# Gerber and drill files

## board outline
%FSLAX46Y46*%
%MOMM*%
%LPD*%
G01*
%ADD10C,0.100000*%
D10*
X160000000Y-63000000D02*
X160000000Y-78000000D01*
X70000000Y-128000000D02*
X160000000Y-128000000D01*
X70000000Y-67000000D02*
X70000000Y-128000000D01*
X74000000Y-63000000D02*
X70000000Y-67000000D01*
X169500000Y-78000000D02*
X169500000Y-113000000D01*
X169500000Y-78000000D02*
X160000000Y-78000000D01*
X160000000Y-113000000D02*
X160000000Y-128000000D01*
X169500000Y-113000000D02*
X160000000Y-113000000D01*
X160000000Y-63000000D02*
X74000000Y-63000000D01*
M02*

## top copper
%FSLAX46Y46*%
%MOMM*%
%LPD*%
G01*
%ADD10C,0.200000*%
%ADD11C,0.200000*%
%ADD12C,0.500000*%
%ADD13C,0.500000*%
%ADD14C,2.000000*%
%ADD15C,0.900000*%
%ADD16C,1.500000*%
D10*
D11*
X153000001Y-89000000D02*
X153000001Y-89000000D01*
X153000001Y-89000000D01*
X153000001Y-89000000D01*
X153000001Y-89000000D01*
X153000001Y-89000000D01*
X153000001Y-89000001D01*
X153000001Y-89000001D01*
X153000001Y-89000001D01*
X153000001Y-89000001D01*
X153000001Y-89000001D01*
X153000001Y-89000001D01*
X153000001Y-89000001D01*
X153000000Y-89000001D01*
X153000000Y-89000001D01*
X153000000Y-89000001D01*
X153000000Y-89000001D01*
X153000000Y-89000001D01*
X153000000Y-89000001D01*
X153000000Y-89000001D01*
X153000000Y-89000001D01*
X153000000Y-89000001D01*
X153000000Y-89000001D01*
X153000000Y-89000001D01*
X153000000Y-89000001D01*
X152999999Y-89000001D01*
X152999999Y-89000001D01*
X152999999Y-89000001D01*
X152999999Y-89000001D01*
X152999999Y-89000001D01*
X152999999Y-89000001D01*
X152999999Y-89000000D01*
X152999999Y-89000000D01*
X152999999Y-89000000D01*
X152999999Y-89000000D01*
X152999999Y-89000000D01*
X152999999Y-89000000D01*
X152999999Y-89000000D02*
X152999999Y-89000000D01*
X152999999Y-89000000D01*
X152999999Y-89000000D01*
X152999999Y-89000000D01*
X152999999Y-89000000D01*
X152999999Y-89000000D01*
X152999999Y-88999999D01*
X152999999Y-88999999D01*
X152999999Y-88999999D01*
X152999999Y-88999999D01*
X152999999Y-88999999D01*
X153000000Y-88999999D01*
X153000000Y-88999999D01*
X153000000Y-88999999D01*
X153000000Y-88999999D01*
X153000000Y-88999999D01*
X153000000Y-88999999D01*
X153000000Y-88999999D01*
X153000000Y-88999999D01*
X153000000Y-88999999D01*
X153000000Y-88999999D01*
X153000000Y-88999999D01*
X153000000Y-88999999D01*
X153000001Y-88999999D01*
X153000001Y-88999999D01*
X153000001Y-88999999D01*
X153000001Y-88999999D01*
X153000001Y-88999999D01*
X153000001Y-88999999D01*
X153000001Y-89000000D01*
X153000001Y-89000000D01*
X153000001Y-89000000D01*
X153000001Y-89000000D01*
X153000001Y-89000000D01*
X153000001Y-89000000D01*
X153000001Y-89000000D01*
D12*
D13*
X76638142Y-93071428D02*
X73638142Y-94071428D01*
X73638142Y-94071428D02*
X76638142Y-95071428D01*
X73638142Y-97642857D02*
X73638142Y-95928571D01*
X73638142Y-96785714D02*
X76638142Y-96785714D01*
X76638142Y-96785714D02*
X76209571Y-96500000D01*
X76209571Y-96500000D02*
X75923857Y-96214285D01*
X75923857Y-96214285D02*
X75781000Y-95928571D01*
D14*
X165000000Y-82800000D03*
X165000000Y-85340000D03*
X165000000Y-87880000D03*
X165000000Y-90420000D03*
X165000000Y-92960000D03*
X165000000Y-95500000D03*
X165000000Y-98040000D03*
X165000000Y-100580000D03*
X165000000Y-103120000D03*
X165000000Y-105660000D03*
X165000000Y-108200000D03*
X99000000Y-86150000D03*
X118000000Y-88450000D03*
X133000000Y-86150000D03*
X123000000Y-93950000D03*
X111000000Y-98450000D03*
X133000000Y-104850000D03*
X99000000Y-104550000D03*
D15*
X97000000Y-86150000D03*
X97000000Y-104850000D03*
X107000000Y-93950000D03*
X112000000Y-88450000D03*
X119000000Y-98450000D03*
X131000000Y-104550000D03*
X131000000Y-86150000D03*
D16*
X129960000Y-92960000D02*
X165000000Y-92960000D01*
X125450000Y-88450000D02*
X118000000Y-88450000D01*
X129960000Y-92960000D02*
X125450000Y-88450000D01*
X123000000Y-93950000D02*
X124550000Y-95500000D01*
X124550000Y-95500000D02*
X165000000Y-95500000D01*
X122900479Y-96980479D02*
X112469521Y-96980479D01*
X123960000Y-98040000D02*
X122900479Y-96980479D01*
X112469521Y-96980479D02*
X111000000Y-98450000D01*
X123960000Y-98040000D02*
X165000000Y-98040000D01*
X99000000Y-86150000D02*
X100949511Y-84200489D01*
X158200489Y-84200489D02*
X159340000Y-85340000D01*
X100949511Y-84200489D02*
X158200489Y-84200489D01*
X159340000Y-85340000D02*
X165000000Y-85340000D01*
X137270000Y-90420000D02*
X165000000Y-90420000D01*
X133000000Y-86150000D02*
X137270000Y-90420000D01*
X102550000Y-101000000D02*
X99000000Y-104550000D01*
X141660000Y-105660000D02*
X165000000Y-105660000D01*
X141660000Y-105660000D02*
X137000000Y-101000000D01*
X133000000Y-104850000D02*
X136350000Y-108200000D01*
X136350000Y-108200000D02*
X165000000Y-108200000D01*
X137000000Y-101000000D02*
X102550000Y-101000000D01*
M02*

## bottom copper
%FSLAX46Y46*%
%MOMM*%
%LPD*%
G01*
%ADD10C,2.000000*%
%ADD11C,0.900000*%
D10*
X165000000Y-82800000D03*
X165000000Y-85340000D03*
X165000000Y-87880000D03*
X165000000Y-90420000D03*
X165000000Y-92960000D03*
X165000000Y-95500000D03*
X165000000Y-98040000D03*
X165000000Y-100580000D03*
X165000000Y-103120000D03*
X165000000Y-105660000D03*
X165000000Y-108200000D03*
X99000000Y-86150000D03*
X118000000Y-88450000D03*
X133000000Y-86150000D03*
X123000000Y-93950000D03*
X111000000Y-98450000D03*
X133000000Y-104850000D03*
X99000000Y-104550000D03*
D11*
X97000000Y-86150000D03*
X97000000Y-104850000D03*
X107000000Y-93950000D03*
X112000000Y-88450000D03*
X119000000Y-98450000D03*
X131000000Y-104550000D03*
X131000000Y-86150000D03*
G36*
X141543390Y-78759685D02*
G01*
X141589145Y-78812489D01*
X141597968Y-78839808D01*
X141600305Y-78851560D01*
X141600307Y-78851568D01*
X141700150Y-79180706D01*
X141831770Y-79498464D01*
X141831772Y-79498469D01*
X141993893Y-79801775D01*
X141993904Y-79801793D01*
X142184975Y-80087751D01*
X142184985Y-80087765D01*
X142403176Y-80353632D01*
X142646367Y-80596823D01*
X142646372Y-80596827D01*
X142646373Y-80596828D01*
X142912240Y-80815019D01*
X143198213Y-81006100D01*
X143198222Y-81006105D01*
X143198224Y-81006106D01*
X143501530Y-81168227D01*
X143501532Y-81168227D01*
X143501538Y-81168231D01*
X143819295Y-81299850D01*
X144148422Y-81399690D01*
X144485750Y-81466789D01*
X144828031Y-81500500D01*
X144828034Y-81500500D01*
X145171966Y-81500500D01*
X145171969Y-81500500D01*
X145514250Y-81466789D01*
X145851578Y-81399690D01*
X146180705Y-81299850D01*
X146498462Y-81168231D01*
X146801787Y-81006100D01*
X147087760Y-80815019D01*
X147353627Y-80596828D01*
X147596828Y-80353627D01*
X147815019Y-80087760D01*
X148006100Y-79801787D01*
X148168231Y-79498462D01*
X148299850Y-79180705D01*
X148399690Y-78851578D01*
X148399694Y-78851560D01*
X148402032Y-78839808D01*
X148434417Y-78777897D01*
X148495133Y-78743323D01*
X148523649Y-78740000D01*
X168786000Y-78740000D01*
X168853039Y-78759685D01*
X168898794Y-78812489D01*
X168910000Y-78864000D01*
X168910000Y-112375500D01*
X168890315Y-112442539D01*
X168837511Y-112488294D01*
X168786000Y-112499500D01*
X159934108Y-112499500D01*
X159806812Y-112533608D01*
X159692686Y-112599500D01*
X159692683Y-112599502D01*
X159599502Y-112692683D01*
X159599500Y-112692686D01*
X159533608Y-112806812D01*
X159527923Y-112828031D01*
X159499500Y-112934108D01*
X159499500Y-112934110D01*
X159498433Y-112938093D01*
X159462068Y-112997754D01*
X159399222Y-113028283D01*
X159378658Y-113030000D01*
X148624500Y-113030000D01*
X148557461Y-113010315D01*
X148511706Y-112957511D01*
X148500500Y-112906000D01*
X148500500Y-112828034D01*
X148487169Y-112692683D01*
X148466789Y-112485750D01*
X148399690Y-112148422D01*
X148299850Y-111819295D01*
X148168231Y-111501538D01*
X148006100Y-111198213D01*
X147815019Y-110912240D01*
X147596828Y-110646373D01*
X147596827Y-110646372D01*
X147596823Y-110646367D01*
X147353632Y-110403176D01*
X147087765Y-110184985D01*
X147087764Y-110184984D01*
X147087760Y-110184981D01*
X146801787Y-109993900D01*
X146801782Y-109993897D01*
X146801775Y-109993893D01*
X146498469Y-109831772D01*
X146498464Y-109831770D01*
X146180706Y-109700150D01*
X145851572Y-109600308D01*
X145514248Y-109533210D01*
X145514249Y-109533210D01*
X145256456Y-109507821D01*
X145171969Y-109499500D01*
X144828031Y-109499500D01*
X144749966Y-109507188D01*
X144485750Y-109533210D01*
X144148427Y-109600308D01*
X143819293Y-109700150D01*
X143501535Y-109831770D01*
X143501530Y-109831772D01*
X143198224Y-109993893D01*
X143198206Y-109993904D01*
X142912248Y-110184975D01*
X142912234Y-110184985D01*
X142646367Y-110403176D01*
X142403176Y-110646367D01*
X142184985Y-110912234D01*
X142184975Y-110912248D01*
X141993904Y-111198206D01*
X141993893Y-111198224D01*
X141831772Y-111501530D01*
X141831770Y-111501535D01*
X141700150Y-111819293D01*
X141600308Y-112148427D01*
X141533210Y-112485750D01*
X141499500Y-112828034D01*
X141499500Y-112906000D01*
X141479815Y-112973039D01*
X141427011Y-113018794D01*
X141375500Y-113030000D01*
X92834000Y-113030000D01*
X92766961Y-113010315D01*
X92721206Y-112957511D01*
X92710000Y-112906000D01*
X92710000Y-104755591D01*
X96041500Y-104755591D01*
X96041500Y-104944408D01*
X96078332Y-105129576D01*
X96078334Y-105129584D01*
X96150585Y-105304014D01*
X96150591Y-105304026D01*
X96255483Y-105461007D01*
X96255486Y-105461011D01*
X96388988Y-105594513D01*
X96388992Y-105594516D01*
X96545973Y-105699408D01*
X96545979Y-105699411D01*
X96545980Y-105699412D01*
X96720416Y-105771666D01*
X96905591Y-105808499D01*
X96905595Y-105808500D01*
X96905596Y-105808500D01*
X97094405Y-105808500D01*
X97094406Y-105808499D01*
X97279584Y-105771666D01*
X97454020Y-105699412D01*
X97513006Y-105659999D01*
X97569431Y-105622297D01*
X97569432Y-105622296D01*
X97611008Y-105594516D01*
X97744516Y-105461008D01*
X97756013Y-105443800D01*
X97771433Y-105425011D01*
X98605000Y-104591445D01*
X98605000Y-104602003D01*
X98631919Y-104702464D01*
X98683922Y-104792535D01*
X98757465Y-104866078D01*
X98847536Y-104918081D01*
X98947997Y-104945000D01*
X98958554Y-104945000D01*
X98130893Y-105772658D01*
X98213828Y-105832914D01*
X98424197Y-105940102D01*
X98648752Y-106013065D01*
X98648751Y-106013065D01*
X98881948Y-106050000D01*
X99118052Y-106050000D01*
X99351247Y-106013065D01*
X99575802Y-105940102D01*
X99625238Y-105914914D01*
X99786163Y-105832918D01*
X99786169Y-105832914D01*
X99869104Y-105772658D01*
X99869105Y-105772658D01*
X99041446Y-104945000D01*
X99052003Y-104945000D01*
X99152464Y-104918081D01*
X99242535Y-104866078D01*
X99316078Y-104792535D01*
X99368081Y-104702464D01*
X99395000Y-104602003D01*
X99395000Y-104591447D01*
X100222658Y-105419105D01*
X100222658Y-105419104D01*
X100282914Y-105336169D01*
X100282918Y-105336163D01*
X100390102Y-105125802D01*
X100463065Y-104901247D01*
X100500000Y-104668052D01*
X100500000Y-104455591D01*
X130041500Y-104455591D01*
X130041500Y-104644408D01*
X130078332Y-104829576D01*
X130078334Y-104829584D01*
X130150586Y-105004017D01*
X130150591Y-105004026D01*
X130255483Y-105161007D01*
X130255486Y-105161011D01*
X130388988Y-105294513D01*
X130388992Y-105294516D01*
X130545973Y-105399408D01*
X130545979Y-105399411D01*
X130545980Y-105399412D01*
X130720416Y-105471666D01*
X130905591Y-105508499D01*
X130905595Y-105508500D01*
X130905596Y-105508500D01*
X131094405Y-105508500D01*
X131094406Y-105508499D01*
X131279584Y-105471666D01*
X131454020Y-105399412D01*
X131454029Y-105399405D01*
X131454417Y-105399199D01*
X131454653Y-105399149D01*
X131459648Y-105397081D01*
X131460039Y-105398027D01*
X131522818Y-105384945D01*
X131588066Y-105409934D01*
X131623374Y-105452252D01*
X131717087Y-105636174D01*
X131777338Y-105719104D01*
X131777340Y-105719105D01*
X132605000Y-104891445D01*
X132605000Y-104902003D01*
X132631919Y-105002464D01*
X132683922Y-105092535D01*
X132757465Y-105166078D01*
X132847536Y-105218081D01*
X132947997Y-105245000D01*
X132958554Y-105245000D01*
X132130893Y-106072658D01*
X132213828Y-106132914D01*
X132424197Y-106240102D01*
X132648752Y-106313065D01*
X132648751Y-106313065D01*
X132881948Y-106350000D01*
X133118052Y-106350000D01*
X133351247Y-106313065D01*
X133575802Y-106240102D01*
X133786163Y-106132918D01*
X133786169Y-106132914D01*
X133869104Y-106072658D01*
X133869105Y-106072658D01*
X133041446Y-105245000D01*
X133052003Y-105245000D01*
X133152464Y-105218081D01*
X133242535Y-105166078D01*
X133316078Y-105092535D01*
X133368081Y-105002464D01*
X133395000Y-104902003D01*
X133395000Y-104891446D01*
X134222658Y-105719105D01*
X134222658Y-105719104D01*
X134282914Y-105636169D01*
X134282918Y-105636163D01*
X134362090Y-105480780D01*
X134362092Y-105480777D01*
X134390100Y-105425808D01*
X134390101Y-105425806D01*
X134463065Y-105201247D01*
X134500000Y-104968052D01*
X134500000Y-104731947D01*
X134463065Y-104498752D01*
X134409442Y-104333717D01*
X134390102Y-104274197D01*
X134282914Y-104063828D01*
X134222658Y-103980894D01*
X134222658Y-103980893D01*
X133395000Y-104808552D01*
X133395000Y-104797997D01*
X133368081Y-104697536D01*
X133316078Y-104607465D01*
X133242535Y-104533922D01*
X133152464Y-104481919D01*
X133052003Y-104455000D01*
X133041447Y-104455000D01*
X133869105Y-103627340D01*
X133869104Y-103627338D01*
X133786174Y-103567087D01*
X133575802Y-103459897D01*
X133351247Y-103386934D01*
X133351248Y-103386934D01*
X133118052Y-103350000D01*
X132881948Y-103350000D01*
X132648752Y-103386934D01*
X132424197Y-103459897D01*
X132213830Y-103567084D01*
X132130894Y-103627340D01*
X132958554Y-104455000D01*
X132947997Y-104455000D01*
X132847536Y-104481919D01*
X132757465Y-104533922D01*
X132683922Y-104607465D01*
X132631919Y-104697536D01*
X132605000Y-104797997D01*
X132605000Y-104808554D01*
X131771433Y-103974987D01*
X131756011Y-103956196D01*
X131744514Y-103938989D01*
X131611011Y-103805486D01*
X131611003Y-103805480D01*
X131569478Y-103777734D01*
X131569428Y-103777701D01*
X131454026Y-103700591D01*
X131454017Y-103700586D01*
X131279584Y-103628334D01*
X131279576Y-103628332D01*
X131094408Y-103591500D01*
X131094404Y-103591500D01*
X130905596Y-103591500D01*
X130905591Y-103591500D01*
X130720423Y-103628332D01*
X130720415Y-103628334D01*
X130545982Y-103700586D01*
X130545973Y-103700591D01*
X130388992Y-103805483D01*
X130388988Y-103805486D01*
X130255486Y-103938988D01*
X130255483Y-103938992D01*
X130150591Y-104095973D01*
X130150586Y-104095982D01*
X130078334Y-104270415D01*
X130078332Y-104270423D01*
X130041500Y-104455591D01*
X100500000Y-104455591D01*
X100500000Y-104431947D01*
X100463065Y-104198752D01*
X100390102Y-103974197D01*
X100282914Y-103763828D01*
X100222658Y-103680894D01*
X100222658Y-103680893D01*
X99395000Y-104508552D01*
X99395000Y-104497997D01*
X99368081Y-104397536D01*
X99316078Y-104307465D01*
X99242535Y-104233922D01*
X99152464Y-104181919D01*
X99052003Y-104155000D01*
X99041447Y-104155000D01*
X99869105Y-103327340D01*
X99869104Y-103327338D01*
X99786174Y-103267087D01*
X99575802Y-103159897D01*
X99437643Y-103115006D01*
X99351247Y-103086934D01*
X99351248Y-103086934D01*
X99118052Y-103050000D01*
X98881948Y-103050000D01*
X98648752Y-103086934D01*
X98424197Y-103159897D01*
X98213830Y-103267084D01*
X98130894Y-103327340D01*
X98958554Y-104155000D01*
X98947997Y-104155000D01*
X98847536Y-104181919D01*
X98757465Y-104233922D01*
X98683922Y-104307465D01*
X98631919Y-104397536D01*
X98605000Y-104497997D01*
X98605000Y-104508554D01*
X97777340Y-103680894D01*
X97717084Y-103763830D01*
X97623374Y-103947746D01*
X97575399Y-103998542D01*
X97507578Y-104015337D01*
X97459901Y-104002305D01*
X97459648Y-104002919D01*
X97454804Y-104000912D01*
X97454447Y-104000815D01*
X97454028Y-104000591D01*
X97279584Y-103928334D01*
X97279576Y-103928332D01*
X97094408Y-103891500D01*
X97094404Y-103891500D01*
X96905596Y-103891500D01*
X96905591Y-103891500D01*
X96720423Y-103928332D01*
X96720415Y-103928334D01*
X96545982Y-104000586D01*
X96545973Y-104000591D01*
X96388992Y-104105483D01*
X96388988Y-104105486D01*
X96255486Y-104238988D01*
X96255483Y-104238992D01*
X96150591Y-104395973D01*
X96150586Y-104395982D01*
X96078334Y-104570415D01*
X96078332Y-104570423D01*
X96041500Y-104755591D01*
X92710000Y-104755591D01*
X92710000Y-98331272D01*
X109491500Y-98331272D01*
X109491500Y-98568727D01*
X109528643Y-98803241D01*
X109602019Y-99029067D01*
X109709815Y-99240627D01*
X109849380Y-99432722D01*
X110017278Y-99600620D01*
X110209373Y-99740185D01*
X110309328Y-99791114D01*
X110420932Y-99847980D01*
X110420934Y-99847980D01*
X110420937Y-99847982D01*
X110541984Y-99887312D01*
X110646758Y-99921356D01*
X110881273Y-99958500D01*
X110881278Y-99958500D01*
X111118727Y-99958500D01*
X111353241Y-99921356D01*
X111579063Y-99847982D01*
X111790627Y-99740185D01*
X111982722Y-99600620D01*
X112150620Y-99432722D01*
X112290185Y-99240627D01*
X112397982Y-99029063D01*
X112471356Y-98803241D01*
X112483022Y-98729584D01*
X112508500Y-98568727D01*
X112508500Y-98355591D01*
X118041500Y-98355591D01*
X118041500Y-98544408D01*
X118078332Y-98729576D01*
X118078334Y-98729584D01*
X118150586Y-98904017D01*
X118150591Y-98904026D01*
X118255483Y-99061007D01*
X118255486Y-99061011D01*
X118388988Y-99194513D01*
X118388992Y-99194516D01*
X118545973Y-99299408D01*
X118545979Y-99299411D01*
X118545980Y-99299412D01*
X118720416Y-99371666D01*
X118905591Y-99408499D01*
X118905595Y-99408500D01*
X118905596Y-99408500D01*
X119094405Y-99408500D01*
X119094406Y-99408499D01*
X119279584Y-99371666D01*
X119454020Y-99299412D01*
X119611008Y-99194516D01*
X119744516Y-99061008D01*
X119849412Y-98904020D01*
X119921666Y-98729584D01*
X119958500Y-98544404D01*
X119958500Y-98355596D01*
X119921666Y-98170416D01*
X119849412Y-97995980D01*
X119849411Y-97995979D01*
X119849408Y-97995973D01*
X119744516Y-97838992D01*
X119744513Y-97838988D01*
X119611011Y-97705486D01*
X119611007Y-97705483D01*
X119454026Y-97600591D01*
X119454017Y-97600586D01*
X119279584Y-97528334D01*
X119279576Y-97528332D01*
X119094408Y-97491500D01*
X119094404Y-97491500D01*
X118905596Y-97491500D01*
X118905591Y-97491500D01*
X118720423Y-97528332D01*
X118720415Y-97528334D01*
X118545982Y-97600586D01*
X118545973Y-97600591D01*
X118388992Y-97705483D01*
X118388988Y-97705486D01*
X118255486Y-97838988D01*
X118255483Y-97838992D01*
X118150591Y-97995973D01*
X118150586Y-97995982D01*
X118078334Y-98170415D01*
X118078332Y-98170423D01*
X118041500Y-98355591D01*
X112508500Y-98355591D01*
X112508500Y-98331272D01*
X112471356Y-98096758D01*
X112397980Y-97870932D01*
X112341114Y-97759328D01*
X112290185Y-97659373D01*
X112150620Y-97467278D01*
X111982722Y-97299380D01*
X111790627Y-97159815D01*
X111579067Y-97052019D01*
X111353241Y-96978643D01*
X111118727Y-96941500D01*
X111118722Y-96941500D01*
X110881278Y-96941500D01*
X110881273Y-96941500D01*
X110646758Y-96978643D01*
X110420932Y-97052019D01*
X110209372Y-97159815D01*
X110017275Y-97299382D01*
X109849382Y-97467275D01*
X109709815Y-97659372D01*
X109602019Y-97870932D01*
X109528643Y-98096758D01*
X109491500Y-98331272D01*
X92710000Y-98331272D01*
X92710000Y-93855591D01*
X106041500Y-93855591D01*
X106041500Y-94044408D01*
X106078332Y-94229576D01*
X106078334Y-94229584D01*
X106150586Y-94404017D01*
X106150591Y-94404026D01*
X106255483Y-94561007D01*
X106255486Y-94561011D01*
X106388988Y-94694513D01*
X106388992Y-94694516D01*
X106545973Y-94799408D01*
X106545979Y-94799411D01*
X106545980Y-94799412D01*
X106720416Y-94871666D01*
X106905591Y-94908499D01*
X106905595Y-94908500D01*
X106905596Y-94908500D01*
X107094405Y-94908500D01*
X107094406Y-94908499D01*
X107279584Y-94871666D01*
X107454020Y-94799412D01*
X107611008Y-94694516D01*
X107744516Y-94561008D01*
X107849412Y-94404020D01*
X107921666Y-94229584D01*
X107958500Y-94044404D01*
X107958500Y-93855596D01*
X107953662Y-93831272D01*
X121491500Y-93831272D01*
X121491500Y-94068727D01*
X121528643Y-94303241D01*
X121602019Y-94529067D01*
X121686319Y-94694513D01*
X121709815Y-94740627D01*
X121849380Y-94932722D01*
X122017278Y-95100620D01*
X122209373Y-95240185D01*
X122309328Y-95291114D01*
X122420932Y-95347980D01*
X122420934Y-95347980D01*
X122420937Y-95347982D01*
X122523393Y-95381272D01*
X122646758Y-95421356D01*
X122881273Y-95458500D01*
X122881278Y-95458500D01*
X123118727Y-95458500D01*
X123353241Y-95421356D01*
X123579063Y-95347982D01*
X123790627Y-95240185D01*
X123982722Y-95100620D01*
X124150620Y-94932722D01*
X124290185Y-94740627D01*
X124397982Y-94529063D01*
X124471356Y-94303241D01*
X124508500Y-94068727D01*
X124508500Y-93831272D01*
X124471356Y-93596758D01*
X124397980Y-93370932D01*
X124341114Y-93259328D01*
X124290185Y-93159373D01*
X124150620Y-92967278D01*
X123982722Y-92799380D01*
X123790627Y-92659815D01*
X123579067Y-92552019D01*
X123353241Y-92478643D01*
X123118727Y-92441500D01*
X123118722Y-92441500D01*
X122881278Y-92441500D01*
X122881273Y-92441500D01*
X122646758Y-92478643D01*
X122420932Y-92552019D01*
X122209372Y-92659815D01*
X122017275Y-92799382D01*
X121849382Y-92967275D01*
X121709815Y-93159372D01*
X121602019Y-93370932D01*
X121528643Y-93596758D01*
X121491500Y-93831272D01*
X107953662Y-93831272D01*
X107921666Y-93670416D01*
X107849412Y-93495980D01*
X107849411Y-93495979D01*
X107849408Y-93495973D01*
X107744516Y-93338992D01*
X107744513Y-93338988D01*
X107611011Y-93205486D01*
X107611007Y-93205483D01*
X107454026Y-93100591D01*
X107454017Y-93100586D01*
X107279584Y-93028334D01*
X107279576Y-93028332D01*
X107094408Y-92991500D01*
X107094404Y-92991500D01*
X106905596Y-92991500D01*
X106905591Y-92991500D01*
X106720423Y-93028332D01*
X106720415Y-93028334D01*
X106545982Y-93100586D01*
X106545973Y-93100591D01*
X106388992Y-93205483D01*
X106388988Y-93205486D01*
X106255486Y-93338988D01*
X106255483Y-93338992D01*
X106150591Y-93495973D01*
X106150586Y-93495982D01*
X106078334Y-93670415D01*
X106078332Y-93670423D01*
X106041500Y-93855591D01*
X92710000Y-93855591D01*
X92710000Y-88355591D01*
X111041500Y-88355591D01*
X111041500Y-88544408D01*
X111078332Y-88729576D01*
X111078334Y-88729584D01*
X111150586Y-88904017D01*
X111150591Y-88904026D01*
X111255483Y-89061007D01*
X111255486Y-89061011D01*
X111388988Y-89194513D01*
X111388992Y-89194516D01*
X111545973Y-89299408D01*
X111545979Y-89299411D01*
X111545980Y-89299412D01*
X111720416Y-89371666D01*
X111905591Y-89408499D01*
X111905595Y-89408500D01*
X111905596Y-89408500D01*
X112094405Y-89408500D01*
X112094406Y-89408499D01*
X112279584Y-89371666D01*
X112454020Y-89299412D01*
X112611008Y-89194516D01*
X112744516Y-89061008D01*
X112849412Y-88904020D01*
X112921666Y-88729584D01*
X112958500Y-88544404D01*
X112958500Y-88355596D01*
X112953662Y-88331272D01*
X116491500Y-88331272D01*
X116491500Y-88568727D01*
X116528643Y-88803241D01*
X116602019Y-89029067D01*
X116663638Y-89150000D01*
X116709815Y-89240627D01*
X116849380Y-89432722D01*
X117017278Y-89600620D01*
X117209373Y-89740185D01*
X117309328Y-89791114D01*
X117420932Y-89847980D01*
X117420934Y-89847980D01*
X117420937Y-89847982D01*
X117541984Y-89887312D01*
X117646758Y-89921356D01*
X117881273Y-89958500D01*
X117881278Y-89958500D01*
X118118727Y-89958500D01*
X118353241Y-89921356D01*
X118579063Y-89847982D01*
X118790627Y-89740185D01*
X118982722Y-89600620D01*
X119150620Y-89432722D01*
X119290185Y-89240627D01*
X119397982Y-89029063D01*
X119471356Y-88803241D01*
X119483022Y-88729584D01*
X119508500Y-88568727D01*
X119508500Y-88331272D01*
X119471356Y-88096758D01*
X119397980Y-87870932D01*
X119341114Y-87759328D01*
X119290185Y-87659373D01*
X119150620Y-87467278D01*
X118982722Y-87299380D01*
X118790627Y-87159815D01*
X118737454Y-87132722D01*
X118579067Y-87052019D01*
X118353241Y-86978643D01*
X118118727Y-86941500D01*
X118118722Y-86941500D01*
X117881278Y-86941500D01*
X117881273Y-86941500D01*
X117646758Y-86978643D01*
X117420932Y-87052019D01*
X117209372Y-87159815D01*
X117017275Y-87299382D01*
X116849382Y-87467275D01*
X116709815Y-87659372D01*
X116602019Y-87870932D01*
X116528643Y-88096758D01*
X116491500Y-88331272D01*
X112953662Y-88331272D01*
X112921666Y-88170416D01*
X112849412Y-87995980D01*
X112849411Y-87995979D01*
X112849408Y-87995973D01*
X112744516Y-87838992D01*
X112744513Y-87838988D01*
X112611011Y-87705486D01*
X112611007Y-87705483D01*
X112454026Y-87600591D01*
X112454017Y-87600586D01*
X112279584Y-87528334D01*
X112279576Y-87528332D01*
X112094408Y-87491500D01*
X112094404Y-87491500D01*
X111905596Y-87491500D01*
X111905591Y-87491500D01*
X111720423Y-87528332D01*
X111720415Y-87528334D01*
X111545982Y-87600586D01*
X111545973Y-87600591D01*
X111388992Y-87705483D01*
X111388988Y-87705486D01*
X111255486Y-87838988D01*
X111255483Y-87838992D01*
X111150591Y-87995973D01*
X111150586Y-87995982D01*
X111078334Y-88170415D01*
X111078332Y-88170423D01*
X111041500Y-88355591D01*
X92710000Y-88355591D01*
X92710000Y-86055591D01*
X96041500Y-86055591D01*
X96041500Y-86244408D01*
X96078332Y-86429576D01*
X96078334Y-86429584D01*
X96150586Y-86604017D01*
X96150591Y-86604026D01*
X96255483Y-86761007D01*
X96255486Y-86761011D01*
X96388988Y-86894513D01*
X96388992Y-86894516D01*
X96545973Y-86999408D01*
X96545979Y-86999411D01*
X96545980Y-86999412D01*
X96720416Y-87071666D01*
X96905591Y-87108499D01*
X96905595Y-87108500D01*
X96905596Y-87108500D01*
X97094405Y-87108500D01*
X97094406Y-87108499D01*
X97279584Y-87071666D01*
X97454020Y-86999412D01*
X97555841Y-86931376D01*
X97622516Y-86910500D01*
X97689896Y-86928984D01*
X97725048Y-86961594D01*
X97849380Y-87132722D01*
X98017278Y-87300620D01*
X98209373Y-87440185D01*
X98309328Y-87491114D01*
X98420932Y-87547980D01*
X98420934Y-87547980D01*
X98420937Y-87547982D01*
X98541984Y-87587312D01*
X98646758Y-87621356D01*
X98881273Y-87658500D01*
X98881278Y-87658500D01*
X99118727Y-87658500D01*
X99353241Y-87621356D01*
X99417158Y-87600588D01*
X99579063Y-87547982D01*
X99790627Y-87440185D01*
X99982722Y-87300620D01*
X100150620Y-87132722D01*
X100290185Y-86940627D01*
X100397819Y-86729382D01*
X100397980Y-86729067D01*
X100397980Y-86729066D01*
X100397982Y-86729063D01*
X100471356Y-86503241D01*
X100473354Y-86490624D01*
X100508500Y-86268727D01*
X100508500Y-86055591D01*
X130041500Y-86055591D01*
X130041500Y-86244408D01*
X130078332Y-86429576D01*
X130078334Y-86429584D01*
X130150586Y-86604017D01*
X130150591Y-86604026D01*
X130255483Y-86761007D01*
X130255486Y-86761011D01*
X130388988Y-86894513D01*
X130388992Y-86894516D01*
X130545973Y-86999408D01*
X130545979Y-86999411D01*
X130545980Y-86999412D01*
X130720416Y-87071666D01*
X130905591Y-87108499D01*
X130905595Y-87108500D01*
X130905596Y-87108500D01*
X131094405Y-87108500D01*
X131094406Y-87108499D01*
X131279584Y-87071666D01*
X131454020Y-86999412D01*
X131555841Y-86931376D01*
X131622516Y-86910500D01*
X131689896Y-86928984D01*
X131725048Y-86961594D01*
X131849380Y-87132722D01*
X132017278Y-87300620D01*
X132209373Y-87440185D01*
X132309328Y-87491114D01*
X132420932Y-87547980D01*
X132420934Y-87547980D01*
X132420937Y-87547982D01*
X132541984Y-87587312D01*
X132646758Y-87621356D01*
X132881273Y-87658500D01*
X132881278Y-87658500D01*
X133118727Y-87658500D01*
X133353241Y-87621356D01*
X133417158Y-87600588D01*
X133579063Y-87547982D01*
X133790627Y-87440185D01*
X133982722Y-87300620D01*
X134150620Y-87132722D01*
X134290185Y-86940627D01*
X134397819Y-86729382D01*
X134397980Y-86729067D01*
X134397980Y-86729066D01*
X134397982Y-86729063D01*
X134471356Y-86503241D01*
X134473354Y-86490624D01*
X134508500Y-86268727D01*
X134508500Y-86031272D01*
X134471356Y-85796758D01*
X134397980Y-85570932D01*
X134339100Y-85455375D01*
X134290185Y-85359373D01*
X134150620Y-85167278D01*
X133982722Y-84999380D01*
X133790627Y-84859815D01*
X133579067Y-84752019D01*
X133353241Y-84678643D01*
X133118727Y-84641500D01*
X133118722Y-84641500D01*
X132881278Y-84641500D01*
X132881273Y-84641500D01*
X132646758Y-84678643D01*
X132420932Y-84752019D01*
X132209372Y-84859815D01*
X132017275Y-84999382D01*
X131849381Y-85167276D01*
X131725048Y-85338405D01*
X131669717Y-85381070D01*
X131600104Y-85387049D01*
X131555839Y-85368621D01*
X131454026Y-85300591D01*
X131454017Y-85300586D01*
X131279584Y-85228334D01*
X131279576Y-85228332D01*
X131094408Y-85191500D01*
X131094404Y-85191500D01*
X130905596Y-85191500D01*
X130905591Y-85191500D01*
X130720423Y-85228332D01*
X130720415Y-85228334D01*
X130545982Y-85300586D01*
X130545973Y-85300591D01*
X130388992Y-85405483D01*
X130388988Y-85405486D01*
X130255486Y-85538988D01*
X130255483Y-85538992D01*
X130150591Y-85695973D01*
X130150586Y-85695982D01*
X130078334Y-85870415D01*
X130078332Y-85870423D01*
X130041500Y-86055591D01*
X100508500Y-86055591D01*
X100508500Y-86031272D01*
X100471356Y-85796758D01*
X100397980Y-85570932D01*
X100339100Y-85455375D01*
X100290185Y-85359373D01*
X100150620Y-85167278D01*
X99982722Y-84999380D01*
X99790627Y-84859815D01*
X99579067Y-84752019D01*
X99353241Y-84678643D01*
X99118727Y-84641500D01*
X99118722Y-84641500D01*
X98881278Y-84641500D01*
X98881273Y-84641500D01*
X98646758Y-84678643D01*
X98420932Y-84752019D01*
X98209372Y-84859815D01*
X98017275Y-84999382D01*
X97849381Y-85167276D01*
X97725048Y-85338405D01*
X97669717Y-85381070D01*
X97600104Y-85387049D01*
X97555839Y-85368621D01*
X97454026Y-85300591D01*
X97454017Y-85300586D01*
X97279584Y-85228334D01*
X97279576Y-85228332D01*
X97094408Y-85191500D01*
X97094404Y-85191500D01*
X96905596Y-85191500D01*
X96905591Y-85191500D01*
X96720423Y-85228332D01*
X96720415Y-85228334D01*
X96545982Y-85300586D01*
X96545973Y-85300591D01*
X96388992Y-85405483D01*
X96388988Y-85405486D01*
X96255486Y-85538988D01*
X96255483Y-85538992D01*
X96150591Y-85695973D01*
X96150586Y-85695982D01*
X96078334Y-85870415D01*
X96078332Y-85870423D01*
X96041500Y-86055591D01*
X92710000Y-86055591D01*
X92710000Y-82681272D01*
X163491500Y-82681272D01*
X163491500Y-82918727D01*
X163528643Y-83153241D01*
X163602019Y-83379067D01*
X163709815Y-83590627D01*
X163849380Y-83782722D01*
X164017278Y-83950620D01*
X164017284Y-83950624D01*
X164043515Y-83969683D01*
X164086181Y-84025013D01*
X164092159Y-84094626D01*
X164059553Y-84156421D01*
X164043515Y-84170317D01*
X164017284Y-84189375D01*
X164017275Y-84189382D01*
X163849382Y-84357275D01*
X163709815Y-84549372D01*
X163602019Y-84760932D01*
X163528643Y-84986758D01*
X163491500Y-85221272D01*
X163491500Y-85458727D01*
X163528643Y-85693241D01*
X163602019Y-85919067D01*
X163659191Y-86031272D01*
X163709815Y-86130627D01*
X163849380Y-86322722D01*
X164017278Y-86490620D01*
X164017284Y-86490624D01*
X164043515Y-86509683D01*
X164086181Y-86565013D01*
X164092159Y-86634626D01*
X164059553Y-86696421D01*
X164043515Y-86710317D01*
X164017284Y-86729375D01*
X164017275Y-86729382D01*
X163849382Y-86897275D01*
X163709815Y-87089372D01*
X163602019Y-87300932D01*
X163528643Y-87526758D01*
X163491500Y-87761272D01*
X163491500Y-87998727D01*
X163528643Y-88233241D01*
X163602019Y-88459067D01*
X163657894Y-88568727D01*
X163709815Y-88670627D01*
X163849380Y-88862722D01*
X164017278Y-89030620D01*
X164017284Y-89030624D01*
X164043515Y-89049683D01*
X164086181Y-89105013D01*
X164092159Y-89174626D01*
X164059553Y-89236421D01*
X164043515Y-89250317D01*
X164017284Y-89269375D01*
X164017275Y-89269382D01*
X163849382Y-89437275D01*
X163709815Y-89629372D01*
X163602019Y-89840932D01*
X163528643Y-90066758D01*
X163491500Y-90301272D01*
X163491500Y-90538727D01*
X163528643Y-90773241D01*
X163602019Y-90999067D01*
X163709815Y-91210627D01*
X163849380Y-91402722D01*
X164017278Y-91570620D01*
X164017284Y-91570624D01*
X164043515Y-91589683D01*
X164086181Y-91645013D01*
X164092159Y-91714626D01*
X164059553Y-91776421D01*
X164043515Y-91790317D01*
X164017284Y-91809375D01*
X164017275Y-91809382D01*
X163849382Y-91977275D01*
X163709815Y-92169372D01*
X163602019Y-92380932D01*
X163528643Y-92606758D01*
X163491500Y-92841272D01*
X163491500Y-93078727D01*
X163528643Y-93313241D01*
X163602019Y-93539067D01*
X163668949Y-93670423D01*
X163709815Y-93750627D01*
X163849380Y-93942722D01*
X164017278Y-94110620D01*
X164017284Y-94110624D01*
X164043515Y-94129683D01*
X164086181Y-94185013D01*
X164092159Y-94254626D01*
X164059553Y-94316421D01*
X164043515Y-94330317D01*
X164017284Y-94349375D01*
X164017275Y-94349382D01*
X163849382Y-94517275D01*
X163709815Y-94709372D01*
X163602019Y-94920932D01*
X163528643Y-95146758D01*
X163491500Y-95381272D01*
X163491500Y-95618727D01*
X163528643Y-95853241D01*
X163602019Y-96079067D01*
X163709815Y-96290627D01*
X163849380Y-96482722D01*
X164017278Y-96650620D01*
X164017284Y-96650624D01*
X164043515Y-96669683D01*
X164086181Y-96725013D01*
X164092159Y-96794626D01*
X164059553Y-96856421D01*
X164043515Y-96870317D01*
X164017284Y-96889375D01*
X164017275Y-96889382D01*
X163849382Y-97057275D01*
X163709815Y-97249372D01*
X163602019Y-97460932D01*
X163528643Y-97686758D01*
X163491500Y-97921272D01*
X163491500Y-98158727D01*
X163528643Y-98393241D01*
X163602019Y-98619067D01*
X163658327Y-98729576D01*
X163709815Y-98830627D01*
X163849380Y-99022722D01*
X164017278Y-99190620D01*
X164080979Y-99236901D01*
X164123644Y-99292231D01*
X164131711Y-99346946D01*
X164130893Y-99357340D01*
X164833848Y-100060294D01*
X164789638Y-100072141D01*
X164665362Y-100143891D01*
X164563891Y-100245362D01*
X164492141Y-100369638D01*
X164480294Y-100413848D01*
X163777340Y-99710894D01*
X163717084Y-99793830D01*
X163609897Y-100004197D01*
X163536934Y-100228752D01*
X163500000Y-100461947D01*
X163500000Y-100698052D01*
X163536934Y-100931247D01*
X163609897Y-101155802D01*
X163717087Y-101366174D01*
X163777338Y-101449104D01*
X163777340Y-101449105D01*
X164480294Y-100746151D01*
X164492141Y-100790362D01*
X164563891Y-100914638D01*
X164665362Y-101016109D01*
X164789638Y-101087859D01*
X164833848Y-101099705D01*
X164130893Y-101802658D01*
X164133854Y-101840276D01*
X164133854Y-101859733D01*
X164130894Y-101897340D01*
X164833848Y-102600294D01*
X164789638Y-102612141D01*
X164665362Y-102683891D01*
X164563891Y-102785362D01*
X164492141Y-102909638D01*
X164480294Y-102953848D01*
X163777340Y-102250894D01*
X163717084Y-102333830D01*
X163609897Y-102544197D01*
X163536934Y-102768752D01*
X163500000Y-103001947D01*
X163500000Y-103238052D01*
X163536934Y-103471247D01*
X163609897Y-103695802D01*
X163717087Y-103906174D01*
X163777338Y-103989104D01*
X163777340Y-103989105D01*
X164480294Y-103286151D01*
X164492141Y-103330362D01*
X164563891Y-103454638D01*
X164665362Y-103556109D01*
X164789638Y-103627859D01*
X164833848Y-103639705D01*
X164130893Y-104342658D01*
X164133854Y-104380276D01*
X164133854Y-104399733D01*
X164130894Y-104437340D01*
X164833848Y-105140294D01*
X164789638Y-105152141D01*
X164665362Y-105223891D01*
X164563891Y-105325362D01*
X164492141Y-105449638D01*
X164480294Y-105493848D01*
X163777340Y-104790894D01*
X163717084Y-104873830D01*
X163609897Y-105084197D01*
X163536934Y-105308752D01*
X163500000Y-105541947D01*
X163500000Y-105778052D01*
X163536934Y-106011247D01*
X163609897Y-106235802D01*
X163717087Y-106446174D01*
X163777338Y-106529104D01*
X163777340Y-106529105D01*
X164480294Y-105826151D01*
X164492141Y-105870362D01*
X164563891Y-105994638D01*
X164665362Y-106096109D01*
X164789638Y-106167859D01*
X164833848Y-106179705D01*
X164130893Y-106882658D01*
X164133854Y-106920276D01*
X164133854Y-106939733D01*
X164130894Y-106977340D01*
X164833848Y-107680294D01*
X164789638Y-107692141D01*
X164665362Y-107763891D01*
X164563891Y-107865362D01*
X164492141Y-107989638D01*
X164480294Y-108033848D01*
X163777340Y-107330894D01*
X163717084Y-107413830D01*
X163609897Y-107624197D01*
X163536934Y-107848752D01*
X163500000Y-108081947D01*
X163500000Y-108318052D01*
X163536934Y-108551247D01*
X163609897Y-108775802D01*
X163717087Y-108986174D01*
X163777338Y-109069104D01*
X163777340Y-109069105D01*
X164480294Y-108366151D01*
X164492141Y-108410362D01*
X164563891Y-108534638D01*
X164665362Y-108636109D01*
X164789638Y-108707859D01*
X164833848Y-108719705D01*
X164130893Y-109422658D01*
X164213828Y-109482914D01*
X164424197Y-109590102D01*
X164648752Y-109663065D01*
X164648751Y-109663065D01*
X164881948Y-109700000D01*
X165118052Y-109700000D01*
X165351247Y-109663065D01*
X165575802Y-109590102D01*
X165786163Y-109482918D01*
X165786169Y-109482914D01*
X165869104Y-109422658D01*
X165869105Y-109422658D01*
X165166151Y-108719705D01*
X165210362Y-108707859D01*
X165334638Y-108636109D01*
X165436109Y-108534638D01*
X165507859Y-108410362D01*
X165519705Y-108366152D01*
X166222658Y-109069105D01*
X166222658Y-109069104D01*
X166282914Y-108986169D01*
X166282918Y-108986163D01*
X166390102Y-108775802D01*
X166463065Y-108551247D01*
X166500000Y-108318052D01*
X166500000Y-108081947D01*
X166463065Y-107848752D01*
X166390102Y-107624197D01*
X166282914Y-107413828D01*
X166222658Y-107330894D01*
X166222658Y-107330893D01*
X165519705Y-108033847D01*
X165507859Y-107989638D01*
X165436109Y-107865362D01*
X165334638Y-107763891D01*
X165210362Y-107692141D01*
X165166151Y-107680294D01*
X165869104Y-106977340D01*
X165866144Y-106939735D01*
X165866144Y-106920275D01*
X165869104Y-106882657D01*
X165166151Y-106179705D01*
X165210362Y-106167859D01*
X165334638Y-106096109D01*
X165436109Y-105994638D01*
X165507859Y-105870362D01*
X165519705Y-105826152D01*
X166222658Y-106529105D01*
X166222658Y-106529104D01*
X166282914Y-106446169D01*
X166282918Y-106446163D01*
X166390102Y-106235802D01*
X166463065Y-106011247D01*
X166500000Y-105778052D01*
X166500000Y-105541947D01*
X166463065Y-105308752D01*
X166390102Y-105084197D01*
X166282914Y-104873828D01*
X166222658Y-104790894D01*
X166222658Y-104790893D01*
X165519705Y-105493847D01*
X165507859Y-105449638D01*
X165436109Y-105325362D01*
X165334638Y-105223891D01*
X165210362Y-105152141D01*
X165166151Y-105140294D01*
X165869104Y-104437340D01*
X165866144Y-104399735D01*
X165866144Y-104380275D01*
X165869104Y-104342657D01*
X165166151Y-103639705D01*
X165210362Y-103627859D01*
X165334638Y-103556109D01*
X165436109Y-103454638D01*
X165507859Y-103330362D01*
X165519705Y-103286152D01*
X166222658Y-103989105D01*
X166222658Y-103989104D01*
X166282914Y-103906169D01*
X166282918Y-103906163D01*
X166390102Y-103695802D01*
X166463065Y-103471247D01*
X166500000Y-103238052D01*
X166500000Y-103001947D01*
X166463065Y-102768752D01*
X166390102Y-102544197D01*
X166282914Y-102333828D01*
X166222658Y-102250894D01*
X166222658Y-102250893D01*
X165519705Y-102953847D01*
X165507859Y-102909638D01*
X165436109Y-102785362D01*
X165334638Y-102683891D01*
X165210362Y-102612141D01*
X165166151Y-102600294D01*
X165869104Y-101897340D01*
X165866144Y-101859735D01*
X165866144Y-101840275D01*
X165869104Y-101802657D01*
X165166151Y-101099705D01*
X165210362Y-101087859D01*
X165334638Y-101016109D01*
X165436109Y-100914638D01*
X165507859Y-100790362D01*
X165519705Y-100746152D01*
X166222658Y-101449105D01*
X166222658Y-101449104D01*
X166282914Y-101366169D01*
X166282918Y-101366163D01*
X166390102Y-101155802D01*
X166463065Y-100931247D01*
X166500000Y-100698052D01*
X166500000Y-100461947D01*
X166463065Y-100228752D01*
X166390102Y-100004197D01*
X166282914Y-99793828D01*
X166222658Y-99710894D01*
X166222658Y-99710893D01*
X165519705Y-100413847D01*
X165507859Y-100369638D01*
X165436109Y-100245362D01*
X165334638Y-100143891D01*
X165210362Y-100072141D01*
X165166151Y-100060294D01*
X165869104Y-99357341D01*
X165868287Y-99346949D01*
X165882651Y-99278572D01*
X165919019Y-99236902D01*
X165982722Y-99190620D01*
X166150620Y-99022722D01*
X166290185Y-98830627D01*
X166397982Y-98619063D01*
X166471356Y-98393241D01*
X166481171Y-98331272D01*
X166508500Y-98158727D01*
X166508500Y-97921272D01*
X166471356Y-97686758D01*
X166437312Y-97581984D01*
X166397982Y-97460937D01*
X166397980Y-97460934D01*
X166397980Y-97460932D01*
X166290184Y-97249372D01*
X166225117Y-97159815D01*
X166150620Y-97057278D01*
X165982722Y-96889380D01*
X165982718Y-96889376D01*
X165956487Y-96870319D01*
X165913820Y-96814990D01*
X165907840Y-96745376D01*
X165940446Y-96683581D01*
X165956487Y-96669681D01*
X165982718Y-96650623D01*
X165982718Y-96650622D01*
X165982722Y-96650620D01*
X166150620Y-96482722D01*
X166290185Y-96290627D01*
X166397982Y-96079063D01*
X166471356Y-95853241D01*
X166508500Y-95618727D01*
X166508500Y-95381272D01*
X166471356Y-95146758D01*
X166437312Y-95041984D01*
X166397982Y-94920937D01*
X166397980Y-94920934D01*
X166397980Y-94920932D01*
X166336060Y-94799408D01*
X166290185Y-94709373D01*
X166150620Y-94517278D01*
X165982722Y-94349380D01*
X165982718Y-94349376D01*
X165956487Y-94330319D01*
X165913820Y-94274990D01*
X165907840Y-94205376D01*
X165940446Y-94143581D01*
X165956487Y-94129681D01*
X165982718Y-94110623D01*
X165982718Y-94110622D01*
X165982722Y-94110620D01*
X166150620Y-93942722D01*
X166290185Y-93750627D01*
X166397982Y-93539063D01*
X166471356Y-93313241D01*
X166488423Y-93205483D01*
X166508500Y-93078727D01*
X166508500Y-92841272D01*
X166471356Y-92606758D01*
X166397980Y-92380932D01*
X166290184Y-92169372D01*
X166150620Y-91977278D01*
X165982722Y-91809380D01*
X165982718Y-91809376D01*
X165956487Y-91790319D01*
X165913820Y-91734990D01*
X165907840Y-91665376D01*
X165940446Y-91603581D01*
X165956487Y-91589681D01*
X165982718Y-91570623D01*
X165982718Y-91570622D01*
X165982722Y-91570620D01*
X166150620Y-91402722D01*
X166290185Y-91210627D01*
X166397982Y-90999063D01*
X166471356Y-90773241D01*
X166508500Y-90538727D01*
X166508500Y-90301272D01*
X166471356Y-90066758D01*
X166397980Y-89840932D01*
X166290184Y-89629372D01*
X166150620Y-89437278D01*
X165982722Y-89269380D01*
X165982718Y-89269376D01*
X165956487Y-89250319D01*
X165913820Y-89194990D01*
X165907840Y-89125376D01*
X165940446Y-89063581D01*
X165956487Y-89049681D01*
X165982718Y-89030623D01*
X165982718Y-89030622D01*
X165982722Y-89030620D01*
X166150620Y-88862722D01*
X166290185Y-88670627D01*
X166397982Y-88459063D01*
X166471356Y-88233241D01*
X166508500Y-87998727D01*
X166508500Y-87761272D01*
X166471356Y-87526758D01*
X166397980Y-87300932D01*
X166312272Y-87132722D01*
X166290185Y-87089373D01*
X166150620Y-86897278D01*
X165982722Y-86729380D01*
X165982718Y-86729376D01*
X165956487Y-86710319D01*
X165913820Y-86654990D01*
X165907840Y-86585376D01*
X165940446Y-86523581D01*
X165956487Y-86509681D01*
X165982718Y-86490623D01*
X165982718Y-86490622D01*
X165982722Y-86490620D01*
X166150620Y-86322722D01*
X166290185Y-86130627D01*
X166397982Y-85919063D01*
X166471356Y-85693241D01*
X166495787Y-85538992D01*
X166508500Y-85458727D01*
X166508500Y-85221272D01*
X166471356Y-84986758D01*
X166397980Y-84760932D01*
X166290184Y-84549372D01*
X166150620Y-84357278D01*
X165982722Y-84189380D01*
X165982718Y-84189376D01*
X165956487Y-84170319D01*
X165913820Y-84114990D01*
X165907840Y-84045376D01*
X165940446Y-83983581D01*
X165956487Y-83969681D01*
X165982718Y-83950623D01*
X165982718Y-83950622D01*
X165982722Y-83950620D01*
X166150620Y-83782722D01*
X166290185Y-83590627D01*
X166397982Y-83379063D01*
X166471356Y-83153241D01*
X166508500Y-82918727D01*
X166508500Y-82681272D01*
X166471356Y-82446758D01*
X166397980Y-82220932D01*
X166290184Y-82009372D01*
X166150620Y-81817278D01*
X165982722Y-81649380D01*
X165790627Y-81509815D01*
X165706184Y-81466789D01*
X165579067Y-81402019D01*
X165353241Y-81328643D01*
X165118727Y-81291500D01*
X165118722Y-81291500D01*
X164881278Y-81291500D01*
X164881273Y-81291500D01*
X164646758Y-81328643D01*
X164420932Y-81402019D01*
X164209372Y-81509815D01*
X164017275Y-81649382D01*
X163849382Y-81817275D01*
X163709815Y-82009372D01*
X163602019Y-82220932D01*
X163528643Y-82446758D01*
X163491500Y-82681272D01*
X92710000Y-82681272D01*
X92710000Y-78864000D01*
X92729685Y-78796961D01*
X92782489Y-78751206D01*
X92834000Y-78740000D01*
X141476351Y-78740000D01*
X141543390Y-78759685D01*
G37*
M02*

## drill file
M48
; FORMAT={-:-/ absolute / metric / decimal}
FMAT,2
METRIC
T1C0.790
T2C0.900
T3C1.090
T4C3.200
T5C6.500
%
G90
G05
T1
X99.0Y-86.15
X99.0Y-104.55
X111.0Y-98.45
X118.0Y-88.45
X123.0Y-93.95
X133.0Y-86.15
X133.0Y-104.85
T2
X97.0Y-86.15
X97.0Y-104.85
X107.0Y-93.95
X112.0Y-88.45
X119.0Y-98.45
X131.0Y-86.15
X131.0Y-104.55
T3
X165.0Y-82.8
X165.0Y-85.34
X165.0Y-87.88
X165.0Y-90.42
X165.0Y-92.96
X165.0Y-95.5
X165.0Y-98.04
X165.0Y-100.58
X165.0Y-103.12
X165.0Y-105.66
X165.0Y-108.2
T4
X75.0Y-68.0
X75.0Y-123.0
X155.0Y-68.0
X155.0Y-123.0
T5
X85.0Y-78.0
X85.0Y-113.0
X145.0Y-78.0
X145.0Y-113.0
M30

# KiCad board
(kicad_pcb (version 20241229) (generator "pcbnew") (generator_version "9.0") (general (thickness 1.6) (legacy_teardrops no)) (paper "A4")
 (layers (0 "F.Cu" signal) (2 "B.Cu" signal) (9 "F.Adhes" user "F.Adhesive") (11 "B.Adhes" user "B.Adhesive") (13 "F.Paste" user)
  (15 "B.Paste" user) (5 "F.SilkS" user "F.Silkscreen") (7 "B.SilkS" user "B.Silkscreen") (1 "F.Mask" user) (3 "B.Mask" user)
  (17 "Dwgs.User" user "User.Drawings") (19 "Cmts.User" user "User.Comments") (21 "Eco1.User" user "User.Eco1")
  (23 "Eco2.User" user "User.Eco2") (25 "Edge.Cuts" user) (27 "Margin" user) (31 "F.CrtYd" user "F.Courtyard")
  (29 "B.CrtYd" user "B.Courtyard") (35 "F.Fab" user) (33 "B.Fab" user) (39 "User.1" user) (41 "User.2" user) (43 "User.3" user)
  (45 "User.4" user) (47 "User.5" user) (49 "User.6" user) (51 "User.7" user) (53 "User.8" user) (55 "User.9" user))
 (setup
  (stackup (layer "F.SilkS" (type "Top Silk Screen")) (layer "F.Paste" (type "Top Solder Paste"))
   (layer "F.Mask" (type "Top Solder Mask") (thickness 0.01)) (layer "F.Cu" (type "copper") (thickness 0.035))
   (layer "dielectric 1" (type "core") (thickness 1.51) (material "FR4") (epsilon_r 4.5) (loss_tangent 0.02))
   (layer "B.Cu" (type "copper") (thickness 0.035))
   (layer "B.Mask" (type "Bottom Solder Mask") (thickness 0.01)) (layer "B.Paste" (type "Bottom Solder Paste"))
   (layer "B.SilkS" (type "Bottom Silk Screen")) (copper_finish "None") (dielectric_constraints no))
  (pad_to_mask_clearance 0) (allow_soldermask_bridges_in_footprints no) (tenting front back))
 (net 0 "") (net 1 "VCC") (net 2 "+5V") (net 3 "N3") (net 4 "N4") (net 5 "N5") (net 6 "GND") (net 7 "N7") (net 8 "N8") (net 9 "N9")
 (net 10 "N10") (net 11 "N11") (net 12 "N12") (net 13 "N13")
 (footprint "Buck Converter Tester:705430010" (layer "F.Cu") (at 165 95.5 -90)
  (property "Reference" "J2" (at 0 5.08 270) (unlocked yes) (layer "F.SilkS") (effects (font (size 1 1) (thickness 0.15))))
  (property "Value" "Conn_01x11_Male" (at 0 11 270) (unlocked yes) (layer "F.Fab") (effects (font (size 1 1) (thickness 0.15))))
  (pad "1" thru_hole circle (at -12.7 0 270) (size 2 2) (drill 1.09) (layers "*.Cu" "*.Mask") (remove_unused_layers no) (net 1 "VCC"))
  (pad "2" thru_hole circle (at -10.16 0 270) (size 2 2) (drill 1.09) (layers "*.Cu" "*.Mask") (remove_unused_layers no) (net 1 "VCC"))
  (pad "3" thru_hole circle (at -7.62 0 270) (size 2 2) (drill 1.09) (layers "*.Cu" "*.Mask") (remove_unused_layers no) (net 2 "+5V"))
  (pad "4" thru_hole circle (at -5.08 0 270) (size 2 2) (drill 1.09) (layers "*.Cu" "*.Mask") (remove_unused_layers no) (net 2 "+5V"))
  (pad "5" thru_hole circle (at -2.54 0 270) (size 2 2) (drill 1.09) (layers "*.Cu" "*.Mask") (remove_unused_layers no) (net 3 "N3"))
  (pad "6" thru_hole circle (at 0 0 270) (size 2 2) (drill 1.09) (layers "*.Cu" "*.Mask") (remove_unused_layers no) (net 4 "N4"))
  (pad "7" thru_hole circle (at 2.54 0 270) (size 2 2) (drill 1.09) (layers "*.Cu" "*.Mask") (remove_unused_layers no) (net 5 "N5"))
  (pad "8" thru_hole circle (at 5.08 0 270) (size 2 2) (drill 1.09) (layers "*.Cu" "*.Mask") (remove_unused_layers no) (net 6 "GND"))
  (pad "9" thru_hole circle (at 7.62 0 270) (size 2 2) (drill 1.09) (layers "*.Cu" "*.Mask") (remove_unused_layers no) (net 6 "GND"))
  (pad "10" thru_hole circle (at 10.16 0 270) (size 2 2) (drill 1.09) (layers "*.Cu" "*.Mask") (remove_unused_layers no) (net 6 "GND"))
  (pad "11" thru_hole circle (at 12.7 0 270) (size 2 2) (drill 1.09) (layers "*.Cu" "*.Mask") (remove_unused_layers no) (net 6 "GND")))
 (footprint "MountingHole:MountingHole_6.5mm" (layer "F.Cu") (at 145 113)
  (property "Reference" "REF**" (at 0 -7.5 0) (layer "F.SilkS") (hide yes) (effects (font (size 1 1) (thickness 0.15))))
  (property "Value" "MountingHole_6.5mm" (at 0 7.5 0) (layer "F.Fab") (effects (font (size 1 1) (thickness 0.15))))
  (pad "" np_thru_hole circle (at 0 0) (size 6.5 6.5) (drill 6.5) (layers "*.Cu" "*.Mask")))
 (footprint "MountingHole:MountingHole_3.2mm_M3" (layer "F.Cu") (at 75 68)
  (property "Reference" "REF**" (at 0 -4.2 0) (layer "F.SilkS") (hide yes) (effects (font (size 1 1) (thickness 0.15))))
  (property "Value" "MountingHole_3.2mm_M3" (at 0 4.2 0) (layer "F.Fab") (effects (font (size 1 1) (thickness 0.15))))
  (pad "" np_thru_hole circle (at 0 0) (size 3.2 3.2) (drill 3.2) (layers "*.Cu" "*.Mask")))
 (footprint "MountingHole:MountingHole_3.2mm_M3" (layer "F.Cu") (at 75 123)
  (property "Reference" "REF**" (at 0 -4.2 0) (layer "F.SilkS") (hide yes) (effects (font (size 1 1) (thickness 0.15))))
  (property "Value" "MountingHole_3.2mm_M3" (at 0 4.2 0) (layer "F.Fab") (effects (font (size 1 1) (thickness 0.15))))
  (pad "" np_thru_hole circle (at 0 0) (size 3.2 3.2) (drill 3.2) (layers "*.Cu" "*.Mask")))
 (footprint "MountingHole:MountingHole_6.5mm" (layer "F.Cu") (at 85 78)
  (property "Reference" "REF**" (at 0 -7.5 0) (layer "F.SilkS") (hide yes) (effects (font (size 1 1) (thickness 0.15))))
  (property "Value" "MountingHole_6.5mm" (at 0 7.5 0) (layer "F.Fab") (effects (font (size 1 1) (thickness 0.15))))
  (pad "" np_thru_hole circle (at 0 0) (size 6.5 6.5) (drill 6.5) (layers "*.Cu" "*.Mask")))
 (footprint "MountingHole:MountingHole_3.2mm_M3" (layer "F.Cu") (at 155 123)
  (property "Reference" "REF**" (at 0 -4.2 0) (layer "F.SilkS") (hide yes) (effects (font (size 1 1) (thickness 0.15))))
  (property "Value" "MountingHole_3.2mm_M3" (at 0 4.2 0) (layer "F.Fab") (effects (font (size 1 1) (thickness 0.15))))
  (pad "" np_thru_hole circle (at 0 0) (size 3.2 3.2) (drill 3.2) (layers "*.Cu" "*.Mask")))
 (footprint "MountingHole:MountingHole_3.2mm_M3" (layer "F.Cu") (at 155 68)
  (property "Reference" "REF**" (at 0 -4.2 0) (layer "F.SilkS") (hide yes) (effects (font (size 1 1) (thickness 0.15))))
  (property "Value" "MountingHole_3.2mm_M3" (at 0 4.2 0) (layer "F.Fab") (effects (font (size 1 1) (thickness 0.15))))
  (pad "" np_thru_hole circle (at 0 0) (size 3.2 3.2) (drill 3.2) (layers "*.Cu" "*.Mask")))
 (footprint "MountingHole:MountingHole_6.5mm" (layer "F.Cu") (at 85 113)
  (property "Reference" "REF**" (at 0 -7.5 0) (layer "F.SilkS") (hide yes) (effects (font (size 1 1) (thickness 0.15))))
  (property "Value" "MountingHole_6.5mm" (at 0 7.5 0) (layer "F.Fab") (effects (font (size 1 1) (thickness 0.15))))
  (pad "" np_thru_hole circle (at 0 0) (size 6.5 6.5) (drill 6.5) (layers "*.Cu" "*.Mask")))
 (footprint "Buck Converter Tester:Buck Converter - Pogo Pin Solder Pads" (layer "F.Cu") (at 133 86.15 180)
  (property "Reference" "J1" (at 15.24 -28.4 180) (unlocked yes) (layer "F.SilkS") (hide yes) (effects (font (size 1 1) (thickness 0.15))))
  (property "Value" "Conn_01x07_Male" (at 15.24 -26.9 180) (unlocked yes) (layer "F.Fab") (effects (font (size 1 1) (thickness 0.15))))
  (pad "1" thru_hole circle (at 34 0 180) (size 2 2) (drill 0.79) (layers "*.Cu" "*.Mask") (remove_unused_layers no) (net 1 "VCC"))
  (pad "2" thru_hole circle (at 15 -2.3 180) (size 2 2) (drill 0.79) (layers "*.Cu" "*.Mask") (remove_unused_layers no) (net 3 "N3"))
  (pad "3" thru_hole circle (at 0 0 180) (size 2 2) (drill 0.79) (layers "*.Cu" "*.Mask") (remove_unused_layers no) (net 2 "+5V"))
  (pad "4" thru_hole circle (at 10 -7.8 180) (size 2 2) (drill 0.79) (layers "*.Cu" "*.Mask") (remove_unused_layers no) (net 4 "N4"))
  (pad "5" thru_hole circle (at 22 -12.3 180) (size 2 2) (drill 0.79) (layers "*.Cu" "*.Mask") (remove_unused_layers no) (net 5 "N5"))
  (pad "6" thru_hole circle (at 0 -18.7 180) (size 2 2) (drill 0.79) (layers "*.Cu" "*.Mask") (remove_unused_layers no) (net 6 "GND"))
  (pad "7" thru_hole circle (at 34 -18.4 180) (size 2 2) (drill 0.79) (layers "*.Cu" "*.Mask") (remove_unused_layers no) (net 6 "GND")))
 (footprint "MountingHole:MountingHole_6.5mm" (layer "F.Cu") (at 145 78)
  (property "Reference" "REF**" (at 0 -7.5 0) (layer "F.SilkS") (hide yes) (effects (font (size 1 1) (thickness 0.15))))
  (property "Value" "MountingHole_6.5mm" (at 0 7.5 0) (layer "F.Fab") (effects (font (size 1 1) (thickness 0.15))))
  (pad "" np_thru_hole circle (at 0 0) (size 6.5 6.5) (drill 6.5) (layers "*.Cu" "*.Mask")))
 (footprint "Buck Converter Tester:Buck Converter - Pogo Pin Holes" (layer "B.Cu") (at 97 86.15)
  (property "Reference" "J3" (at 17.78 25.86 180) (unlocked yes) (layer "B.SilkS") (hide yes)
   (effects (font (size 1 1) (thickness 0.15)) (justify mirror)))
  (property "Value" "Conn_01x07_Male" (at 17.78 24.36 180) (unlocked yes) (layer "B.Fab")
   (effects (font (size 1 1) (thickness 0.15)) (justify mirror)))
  (pad "1" thru_hole circle (at 0 0) (size 0.9 0.9) (drill 0.9) (layers "*.Cu" "*.Mask") (remove_unused_layers no) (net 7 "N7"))
  (pad "2" thru_hole circle (at 0 18.7) (size 0.9 0.9) (drill 0.9) (layers "*.Cu" "*.Mask") (remove_unused_layers no) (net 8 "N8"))
  (pad "3" thru_hole circle (at 10 7.8) (size 0.9 0.9) (drill 0.9) (layers "*.Cu" "*.Mask") (remove_unused_layers no) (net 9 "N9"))
  (pad "4" thru_hole circle (at 15 2.3) (size 0.9 0.9) (drill 0.9) (layers "*.Cu" "*.Mask") (remove_unused_layers no) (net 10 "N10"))
  (pad "5" thru_hole circle (at 22 12.3) (size 0.9 0.9) (drill 0.9) (layers "*.Cu" "*.Mask") (remove_unused_layers no) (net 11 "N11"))
  (pad "6" thru_hole circle (at 34 18.4) (size 0.9 0.9) (drill 0.9) (layers "*.Cu" "*.Mask") (remove_unused_layers no) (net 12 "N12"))
  (pad "7" thru_hole circle (at 34 0) (size 0.9 0.9) (drill 0.9) (layers "*.Cu" "*.Mask") (remove_unused_layers no) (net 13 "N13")))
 (gr_circle (center 153 89) (end 153 89) (stroke (width 0.2) (type solid)) (fill no) (layer "F.Cu"))
 (gr_line (start 160 63) (end 160 78) (stroke (width 0.1) (type solid)) (layer "Edge.Cuts"))
 (gr_line (start 70 128) (end 160 128) (stroke (width 0.1) (type solid)) (layer "Edge.Cuts"))
 (gr_line (start 70 67) (end 70 128) (stroke (width 0.1) (type solid)) (layer "Edge.Cuts"))
 (gr_line (start 74 63) (end 70 67) (stroke (width 0.1) (type solid)) (layer "Edge.Cuts"))
 (gr_line (start 169.5 78) (end 169.5 113) (stroke (width 0.1) (type solid)) (layer "Edge.Cuts"))
 (gr_line (start 169.5 78) (end 160 78) (stroke (width 0.1) (type solid)) (layer "Edge.Cuts"))
 (gr_line (start 160 113) (end 160 128) (stroke (width 0.1) (type solid)) (layer "Edge.Cuts"))
 (gr_line (start 169.5 113) (end 160 113) (stroke (width 0.1) (type solid)) (layer "Edge.Cuts"))
 (gr_line (start 160 63) (end 74 63) (stroke (width 0.1) (type solid)) (layer "Edge.Cuts"))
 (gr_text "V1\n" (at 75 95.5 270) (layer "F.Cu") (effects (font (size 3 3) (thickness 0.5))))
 (segment (start 129.96 92.96) (end 165 92.96) (width 1.5) (layer "F.Cu") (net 3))
 (segment (start 125.45 88.45) (end 118 88.45) (width 1.5) (layer "F.Cu") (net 3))
 (segment (start 129.96 92.96) (end 125.45 88.45) (width 1.5) (layer "F.Cu") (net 3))
 (segment (start 123 93.95) (end 124.55 95.5) (width 1.5) (layer "F.Cu") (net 4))
 (segment (start 124.55 95.5) (end 165 95.5) (width 1.5) (layer "F.Cu") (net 4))
 (segment (start 122.900479 96.980479) (end 112.469521 96.980479) (width 1.5) (layer "F.Cu") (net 5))
 (segment (start 123.96 98.04) (end 122.900479 96.980479) (width 1.5) (layer "F.Cu") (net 5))
 (segment (start 112.469521 96.980479) (end 111 98.45) (width 1.5) (layer "F.Cu") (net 5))
 (segment (start 123.96 98.04) (end 165 98.04) (width 1.5) (layer "F.Cu") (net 5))
 (segment (start 99 86.15) (end 100.949511 84.200489) (width 1.5) (layer "F.Cu") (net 1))
 (segment (start 158.200489 84.200489) (end 159.34 85.34) (width 1.5) (layer "F.Cu") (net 1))
 (segment (start 100.949511 84.200489) (end 158.200489 84.200489) (width 1.5) (layer "F.Cu") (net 1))
 (segment (start 159.34 85.34) (end 165 85.34) (width 1.5) (layer "F.Cu") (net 1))
 (segment (start 137.27 90.42) (end 165 90.42) (width 1.5) (layer "F.Cu") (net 2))
 (segment (start 133 86.15) (end 137.27 90.42) (width 1.5) (layer "F.Cu") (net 2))
 (segment (start 102.55 101) (end 99 104.55) (width 1.5) (layer "F.Cu") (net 6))
 (segment (start 141.66 105.66) (end 165 105.66) (width 1.5) (layer "F.Cu") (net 6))
 (segment (start 141.66 105.66) (end 137 101) (width 1.5) (layer "F.Cu") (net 6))
 (segment (start 133 104.85) (end 136.35 108.2) (width 1.5) (layer "F.Cu") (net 6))
 (segment (start 136.35 108.2) (end 165 108.2) (width 1.5) (layer "F.Cu") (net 6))
 (segment (start 137 101) (end 102.55 101) (width 1.5) (layer "F.Cu") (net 6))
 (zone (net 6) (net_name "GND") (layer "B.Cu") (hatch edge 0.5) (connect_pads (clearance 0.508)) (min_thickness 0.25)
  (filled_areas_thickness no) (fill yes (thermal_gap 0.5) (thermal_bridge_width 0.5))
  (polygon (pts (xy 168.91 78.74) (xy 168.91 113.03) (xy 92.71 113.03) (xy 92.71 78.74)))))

